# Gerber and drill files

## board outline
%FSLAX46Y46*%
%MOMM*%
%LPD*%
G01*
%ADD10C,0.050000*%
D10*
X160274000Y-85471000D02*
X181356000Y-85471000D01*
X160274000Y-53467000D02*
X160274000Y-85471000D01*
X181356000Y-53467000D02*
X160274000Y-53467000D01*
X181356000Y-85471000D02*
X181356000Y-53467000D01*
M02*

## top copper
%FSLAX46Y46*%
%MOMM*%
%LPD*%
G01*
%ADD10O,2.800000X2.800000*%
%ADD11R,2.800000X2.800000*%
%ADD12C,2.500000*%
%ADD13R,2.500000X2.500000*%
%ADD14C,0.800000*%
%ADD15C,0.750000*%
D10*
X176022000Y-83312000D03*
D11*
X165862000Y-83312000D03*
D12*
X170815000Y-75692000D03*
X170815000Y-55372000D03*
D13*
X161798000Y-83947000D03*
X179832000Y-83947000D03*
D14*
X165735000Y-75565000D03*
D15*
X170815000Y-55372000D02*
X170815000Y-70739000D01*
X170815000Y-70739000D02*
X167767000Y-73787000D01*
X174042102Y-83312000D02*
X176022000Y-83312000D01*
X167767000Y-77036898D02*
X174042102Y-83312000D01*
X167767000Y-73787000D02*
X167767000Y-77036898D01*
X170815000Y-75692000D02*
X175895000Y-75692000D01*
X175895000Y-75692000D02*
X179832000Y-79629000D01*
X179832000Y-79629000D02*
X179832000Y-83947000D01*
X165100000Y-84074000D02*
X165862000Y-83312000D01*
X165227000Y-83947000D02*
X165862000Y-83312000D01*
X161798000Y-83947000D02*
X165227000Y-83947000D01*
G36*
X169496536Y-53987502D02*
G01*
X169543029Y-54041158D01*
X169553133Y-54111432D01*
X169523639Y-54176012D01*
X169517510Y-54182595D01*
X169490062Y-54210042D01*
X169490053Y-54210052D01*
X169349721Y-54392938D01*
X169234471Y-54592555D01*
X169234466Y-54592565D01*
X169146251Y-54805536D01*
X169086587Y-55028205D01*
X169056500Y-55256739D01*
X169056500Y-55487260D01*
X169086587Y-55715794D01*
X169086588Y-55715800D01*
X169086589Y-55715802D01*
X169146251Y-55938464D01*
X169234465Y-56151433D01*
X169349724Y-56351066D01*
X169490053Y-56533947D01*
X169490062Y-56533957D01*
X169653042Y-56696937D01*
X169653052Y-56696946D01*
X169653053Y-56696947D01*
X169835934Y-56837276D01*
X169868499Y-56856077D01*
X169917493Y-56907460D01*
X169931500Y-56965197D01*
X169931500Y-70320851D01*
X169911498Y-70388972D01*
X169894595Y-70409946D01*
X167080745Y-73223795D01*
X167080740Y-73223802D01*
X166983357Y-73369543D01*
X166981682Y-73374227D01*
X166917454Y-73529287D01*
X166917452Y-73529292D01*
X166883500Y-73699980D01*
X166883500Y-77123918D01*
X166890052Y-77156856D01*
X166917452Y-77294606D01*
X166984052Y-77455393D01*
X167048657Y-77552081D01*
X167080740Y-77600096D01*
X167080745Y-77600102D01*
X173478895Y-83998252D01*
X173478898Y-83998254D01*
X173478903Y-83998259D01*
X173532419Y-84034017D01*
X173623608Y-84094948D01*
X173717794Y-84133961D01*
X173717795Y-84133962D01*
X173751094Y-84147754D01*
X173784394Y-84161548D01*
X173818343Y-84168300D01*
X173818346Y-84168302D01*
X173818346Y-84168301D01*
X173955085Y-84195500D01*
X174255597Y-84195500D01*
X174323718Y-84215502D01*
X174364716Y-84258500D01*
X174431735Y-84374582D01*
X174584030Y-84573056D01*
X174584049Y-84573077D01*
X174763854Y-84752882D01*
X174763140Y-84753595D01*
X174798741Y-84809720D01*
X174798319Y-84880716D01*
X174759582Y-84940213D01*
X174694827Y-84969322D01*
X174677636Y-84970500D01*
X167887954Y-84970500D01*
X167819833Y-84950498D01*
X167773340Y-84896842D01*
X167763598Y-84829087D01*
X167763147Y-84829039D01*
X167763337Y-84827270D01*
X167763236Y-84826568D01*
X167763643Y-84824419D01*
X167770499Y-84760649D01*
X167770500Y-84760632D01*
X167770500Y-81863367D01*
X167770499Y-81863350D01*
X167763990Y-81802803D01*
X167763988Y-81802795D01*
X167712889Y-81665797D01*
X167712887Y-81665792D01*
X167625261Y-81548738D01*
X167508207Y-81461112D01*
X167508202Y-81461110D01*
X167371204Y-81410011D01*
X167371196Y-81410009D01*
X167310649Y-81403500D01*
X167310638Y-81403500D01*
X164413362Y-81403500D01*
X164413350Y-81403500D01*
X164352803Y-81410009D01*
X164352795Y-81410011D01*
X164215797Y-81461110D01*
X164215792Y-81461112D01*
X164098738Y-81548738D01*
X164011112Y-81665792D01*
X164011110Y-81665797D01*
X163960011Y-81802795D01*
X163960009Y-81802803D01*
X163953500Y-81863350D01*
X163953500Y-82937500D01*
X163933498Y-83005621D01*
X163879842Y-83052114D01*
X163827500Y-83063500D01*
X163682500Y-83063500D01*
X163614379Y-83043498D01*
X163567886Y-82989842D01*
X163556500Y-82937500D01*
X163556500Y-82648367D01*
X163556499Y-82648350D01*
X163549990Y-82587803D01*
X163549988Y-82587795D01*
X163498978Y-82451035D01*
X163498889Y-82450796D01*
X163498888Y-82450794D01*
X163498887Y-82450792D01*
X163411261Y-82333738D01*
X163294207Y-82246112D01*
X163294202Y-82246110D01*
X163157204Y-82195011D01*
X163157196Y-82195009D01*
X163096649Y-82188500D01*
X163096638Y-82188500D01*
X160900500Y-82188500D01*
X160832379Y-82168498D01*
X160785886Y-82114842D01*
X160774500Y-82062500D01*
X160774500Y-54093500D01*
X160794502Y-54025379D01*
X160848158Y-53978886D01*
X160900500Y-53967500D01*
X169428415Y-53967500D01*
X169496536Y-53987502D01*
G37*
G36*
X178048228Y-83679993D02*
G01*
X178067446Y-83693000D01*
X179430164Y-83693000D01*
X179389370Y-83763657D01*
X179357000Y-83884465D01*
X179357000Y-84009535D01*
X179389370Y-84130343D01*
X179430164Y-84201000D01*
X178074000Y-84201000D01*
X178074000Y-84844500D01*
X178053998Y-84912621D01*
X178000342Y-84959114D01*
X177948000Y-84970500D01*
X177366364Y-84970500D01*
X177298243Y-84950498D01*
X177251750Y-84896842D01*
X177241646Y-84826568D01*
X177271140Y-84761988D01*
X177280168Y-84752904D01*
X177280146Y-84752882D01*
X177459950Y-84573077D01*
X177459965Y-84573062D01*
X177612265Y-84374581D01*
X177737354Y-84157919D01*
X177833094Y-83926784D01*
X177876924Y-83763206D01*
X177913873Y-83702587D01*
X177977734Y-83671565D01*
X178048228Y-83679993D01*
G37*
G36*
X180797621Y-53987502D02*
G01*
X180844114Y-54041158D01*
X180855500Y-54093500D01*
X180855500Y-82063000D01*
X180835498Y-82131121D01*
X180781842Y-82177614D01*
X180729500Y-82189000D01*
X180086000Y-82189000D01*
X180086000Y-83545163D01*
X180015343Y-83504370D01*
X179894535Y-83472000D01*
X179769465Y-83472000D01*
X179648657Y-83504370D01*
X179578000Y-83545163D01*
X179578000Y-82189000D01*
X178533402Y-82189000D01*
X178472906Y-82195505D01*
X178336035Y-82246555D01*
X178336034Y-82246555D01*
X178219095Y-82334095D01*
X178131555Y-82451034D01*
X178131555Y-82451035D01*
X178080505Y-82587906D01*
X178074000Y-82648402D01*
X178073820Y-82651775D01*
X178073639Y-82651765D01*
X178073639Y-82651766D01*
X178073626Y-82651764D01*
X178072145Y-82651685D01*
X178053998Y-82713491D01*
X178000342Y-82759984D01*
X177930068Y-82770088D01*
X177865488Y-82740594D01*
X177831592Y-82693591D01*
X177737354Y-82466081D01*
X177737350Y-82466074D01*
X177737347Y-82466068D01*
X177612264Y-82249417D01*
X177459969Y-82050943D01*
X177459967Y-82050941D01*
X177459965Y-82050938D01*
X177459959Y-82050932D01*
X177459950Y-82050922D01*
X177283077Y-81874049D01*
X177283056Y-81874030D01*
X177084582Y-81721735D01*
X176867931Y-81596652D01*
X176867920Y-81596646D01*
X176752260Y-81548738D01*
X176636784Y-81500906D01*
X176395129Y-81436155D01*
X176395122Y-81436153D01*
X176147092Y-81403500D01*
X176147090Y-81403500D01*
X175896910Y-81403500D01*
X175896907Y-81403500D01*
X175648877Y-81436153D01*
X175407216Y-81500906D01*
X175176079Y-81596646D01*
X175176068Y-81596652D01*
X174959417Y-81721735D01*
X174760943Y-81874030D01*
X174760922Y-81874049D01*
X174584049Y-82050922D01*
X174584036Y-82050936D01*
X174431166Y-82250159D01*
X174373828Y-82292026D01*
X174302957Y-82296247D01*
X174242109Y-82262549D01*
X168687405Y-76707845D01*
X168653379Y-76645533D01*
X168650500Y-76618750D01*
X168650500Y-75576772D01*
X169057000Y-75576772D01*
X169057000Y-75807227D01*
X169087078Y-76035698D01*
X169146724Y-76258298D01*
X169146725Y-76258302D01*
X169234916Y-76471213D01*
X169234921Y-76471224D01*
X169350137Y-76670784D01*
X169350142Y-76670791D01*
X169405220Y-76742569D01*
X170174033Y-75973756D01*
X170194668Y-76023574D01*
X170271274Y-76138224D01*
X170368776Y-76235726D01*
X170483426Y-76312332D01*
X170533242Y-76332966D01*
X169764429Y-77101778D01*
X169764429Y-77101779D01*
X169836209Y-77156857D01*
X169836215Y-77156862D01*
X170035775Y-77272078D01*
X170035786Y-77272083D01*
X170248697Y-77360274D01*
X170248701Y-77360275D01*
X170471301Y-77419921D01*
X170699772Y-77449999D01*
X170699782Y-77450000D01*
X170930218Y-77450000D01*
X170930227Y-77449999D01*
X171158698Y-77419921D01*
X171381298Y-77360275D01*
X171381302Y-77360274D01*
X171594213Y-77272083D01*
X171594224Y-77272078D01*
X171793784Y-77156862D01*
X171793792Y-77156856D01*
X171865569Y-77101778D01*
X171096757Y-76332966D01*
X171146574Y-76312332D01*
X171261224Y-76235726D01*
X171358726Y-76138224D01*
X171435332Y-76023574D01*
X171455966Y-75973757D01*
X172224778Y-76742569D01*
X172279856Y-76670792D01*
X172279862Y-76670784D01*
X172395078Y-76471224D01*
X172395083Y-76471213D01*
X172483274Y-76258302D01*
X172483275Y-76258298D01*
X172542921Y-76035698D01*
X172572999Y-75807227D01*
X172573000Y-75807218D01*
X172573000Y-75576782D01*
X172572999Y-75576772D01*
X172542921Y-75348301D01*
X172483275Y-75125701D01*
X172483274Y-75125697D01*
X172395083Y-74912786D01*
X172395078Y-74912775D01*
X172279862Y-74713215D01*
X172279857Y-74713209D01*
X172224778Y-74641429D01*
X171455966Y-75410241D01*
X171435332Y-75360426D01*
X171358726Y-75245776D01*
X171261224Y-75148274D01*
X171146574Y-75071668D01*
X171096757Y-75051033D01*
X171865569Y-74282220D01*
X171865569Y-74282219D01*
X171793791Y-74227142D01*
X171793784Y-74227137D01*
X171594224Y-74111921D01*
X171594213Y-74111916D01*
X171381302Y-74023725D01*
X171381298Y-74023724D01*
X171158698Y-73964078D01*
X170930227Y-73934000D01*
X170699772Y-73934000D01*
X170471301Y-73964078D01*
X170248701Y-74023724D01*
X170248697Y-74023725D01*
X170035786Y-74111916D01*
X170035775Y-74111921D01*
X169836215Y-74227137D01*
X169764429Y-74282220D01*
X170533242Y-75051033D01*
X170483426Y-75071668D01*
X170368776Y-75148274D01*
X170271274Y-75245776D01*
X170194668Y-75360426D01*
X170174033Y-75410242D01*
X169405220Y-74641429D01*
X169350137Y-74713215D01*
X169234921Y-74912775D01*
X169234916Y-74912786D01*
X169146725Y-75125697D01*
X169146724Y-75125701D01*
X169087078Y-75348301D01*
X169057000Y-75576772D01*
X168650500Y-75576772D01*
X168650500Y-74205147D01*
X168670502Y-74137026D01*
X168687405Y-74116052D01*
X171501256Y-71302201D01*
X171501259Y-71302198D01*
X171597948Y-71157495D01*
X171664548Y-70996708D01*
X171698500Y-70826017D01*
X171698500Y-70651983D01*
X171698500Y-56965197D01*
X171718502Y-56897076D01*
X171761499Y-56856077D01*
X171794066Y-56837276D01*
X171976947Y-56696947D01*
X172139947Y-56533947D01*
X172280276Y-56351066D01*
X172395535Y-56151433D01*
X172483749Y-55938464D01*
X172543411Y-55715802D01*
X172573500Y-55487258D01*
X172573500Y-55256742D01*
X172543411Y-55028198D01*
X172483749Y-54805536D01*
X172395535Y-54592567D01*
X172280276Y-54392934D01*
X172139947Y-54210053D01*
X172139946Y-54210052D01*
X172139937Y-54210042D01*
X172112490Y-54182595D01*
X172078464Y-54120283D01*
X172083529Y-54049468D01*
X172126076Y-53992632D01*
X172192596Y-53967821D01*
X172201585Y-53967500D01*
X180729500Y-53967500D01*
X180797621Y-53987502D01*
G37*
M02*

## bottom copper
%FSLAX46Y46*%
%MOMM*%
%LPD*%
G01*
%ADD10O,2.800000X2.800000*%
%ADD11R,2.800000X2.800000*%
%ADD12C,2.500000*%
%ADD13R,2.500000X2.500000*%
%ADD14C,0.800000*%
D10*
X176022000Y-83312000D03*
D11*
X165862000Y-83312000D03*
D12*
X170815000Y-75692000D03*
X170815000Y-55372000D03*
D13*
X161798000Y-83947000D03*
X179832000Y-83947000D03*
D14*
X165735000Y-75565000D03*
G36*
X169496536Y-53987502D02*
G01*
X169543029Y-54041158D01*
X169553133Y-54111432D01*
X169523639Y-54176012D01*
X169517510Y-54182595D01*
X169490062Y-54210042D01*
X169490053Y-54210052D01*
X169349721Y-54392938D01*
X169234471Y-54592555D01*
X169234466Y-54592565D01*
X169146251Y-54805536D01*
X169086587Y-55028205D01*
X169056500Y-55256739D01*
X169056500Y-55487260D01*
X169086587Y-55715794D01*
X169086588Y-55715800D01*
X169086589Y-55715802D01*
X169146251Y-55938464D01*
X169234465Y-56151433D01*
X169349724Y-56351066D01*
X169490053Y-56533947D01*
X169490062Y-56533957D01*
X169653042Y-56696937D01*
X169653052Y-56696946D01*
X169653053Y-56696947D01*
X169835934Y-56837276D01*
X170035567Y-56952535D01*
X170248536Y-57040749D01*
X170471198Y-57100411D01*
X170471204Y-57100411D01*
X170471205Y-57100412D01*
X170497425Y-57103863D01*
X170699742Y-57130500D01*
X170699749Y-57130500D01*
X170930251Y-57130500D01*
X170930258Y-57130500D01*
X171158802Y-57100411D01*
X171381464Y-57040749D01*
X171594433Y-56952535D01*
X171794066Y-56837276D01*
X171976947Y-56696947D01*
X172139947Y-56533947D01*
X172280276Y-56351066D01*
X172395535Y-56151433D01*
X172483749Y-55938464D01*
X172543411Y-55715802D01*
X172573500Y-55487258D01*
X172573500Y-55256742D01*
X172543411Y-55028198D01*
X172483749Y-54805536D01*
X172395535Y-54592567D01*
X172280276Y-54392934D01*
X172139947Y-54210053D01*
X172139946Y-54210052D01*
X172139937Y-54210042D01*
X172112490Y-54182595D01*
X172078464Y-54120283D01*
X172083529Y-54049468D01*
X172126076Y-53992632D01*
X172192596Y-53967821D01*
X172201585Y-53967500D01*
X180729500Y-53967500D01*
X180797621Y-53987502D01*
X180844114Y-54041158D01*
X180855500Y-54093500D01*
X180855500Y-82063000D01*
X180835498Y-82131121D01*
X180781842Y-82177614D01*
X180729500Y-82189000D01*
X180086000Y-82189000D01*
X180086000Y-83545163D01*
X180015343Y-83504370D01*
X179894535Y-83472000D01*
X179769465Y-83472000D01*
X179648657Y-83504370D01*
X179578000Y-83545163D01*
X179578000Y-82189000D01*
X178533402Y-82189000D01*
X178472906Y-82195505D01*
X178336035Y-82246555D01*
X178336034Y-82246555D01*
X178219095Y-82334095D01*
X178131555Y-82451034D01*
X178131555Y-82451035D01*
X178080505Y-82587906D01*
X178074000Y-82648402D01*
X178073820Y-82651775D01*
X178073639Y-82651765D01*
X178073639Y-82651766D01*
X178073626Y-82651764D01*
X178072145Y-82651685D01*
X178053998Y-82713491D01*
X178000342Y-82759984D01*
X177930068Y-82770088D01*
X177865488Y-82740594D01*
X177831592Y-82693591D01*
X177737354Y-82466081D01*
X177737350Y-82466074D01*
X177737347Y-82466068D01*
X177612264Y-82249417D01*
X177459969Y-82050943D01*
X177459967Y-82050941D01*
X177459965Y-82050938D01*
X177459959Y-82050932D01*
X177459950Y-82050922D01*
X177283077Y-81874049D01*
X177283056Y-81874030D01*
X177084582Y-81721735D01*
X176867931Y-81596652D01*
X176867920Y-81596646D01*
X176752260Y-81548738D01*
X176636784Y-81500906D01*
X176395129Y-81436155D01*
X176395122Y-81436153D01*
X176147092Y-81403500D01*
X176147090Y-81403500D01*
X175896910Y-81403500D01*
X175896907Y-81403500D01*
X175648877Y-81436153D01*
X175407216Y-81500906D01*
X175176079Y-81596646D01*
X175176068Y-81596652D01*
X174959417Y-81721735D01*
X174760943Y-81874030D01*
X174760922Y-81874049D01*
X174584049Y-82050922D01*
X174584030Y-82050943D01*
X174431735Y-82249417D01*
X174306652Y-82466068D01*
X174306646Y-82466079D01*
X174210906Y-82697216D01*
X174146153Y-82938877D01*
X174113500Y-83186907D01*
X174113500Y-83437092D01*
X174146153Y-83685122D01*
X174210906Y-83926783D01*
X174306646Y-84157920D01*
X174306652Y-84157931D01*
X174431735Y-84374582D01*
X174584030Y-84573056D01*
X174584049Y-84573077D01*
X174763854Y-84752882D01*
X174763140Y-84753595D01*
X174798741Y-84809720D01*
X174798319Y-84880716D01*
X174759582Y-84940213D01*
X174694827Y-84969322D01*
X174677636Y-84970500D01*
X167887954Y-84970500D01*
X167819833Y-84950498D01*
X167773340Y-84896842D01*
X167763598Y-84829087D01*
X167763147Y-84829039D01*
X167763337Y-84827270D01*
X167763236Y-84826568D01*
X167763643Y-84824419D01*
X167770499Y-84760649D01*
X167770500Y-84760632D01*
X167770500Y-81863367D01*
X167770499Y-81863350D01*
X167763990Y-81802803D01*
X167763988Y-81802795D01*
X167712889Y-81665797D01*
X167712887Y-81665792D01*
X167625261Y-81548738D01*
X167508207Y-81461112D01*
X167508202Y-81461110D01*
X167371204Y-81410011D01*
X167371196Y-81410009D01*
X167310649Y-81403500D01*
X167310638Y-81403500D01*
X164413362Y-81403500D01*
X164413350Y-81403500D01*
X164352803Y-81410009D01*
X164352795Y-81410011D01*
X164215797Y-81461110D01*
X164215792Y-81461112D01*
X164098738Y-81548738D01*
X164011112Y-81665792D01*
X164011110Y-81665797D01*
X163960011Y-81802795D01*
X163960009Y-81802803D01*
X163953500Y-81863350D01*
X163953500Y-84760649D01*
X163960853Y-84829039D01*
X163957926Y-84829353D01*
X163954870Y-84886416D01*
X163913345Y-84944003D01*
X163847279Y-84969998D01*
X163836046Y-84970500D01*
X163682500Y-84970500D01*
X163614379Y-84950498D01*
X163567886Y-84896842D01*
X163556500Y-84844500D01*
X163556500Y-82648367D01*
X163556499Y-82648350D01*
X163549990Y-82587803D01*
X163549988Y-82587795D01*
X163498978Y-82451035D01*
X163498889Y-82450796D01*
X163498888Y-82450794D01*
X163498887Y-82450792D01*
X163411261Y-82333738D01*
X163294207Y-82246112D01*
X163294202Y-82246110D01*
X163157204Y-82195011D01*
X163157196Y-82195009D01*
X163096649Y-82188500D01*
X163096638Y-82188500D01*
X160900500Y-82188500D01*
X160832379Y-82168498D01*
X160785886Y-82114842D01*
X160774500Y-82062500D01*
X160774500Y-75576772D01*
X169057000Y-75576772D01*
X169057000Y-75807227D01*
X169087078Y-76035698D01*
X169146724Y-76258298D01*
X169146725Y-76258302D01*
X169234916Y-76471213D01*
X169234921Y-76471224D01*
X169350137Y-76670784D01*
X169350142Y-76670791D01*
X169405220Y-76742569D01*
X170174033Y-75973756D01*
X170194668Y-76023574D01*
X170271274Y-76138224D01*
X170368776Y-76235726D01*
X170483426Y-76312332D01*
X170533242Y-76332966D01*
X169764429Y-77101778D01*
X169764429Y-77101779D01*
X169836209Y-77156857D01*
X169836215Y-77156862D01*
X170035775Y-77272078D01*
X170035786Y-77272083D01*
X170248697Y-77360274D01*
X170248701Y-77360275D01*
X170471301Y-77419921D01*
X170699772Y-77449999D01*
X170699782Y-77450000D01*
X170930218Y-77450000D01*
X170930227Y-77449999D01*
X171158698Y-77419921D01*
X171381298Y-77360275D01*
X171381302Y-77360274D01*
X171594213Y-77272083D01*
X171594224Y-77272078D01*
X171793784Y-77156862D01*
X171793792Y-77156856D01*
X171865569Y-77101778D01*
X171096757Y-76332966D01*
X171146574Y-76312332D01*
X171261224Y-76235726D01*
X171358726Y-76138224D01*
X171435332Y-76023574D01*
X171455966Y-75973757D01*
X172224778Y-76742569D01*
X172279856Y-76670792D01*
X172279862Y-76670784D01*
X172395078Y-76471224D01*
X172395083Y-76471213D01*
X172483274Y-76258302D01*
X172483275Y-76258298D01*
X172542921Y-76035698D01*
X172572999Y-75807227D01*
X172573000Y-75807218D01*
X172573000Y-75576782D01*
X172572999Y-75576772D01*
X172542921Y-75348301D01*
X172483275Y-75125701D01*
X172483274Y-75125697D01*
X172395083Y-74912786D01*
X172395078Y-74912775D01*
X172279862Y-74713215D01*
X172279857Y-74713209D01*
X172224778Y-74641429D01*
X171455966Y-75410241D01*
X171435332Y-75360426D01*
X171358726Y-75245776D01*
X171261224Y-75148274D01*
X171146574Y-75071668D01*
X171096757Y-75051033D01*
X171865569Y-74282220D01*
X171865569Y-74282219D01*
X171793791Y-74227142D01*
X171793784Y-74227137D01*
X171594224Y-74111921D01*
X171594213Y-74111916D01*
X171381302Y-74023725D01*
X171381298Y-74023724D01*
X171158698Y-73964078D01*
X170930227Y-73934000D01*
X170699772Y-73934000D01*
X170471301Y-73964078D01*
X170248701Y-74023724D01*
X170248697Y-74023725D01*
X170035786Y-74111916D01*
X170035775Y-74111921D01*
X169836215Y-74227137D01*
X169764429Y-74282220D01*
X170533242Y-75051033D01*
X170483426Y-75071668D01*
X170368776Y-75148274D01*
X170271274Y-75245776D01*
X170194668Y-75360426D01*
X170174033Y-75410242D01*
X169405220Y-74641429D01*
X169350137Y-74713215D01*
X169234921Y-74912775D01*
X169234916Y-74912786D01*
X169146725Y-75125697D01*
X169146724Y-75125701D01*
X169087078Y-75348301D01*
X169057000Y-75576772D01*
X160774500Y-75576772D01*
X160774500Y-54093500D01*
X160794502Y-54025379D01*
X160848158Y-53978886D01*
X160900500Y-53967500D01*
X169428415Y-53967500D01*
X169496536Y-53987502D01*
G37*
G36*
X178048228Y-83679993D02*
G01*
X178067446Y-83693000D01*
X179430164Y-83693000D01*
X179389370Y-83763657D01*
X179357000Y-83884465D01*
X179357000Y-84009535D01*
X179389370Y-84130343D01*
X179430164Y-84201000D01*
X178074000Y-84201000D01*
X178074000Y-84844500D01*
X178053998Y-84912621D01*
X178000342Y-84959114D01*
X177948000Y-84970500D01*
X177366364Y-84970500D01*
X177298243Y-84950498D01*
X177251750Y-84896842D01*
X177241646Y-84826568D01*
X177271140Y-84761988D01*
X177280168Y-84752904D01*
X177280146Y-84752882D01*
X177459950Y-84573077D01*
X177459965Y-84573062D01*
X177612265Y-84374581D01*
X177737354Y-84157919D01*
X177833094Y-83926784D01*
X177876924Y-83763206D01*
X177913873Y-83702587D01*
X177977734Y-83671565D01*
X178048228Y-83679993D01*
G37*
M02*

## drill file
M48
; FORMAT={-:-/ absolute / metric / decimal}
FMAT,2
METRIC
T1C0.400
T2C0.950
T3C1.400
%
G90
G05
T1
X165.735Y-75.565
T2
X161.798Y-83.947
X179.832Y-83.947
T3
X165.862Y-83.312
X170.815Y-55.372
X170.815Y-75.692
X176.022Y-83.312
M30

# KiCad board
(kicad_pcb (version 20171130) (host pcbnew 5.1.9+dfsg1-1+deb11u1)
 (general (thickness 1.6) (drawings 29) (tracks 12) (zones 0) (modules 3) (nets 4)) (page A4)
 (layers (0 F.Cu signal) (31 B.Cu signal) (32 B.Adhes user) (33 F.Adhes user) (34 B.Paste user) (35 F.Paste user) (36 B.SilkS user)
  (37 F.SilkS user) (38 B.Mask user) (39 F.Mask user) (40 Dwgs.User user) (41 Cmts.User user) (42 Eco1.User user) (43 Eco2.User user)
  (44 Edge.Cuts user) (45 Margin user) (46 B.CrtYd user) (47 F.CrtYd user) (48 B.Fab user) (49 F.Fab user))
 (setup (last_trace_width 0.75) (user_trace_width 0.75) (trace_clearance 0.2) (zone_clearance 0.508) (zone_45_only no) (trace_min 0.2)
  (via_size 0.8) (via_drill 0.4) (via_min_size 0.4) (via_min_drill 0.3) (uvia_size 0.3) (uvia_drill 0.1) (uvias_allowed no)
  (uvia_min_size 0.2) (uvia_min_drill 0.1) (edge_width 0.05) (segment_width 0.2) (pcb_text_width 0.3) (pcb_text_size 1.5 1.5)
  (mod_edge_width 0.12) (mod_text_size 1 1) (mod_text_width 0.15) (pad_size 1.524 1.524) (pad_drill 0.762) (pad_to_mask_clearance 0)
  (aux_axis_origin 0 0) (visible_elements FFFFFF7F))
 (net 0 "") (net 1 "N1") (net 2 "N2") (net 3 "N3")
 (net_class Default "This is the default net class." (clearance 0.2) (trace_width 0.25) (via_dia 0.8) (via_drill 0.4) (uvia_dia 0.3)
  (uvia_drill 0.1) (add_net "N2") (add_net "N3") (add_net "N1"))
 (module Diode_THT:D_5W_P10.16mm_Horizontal (layer F.Cu) (at 165.862 83.312)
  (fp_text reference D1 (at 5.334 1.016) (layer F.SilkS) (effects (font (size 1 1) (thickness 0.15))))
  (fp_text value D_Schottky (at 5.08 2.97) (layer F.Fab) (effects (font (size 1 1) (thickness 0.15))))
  (pad 2 thru_hole oval (at 10.16 0) (size 2.8 2.8) (drill 1.4) (layers *.Cu *.Mask) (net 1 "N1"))
  (pad 1 thru_hole rect (at 0 0) (size 2.8 2.8) (drill 1.4) (layers *.Cu *.Mask) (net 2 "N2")))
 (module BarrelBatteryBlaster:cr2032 (layer F.Cu) (at 170.815 55.372 270)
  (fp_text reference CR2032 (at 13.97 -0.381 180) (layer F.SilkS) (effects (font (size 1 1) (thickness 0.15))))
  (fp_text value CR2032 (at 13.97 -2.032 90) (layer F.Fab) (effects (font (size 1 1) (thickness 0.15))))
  (pad 2 thru_hole circle (at 20.32 0 270) (size 2.5 2.5) (drill 1.4) (layers *.Cu *.Mask) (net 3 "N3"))
  (pad 1 thru_hole circle (at 0 0 270) (size 2.5 2.5) (drill 1.4) (layers *.Cu *.Mask) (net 1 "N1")))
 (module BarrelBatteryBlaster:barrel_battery (layer B.Cu) (at 179.832 83.947 180)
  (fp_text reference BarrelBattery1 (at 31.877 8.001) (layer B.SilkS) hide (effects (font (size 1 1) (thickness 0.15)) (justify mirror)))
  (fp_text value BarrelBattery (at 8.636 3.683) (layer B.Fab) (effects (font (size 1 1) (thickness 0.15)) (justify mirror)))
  (pad 1 thru_hole rect (at 18.034 0 180) (size 2.5 2.5) (drill 0.95) (layers *.Cu *.Mask) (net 2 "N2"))
  (pad 2 thru_hole rect (at 0 0 90) (size 2.5 2.5) (drill 0.95) (layers *.Cu *.Mask) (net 3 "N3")))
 (gr_line (start 160.274 85.471) (end 181.356 85.471) (layer Edge.Cuts) (width 0.05))
 (gr_line (start 160.274 53.467) (end 160.274 85.471) (layer Edge.Cuts) (width 0.05))
 (gr_line (start 181.356 53.467) (end 160.274 53.467) (layer Edge.Cuts) (width 0.05))
 (gr_line (start 181.356 85.471) (end 181.356 53.467) (layer Edge.Cuts) (width 0.05))
 (segment (start 170.815 55.372) (end 170.815 70.739) (width 0.75) (layer F.Cu) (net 1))
 (segment (start 170.815 70.739) (end 167.767 73.787) (width 0.75) (layer F.Cu) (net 1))
 (segment (start 174.042102 83.312) (end 176.022 83.312) (width 0.75) (layer F.Cu) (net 1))
 (segment (start 167.767 77.036898) (end 174.042102 83.312) (width 0.75) (layer F.Cu) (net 1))
 (segment (start 167.767 73.787) (end 167.767 77.036898) (width 0.75) (layer F.Cu) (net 1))
 (segment (start 170.815 75.692) (end 175.895 75.692) (width 0.75) (layer F.Cu) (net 3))
 (segment (start 175.895 75.692) (end 179.832 79.629) (width 0.75) (layer F.Cu) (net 3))
 (segment (start 179.832 79.629) (end 179.832 83.947) (width 0.75) (layer F.Cu) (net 3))
 (via (at 165.735 75.565) (size 0.8) (drill 0.4) (layers F.Cu B.Cu) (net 3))
 (segment (start 165.1 84.074) (end 165.862 83.312) (width 0.75) (layer F.Cu) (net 2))
 (segment (start 165.227 83.947) (end 165.862 83.312) (width 0.75) (layer F.Cu) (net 2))
 (segment (start 161.798 83.947) (end 165.227 83.947) (width 0.75) (layer F.Cu) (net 2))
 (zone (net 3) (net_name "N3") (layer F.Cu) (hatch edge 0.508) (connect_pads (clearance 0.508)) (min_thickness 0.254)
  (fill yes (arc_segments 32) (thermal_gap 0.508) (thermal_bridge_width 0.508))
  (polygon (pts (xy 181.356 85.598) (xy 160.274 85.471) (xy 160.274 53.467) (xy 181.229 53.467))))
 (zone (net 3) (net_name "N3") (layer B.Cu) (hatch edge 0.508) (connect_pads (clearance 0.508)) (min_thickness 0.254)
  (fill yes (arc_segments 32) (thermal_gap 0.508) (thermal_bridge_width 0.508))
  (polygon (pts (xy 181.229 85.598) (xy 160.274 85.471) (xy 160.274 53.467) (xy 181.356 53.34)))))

